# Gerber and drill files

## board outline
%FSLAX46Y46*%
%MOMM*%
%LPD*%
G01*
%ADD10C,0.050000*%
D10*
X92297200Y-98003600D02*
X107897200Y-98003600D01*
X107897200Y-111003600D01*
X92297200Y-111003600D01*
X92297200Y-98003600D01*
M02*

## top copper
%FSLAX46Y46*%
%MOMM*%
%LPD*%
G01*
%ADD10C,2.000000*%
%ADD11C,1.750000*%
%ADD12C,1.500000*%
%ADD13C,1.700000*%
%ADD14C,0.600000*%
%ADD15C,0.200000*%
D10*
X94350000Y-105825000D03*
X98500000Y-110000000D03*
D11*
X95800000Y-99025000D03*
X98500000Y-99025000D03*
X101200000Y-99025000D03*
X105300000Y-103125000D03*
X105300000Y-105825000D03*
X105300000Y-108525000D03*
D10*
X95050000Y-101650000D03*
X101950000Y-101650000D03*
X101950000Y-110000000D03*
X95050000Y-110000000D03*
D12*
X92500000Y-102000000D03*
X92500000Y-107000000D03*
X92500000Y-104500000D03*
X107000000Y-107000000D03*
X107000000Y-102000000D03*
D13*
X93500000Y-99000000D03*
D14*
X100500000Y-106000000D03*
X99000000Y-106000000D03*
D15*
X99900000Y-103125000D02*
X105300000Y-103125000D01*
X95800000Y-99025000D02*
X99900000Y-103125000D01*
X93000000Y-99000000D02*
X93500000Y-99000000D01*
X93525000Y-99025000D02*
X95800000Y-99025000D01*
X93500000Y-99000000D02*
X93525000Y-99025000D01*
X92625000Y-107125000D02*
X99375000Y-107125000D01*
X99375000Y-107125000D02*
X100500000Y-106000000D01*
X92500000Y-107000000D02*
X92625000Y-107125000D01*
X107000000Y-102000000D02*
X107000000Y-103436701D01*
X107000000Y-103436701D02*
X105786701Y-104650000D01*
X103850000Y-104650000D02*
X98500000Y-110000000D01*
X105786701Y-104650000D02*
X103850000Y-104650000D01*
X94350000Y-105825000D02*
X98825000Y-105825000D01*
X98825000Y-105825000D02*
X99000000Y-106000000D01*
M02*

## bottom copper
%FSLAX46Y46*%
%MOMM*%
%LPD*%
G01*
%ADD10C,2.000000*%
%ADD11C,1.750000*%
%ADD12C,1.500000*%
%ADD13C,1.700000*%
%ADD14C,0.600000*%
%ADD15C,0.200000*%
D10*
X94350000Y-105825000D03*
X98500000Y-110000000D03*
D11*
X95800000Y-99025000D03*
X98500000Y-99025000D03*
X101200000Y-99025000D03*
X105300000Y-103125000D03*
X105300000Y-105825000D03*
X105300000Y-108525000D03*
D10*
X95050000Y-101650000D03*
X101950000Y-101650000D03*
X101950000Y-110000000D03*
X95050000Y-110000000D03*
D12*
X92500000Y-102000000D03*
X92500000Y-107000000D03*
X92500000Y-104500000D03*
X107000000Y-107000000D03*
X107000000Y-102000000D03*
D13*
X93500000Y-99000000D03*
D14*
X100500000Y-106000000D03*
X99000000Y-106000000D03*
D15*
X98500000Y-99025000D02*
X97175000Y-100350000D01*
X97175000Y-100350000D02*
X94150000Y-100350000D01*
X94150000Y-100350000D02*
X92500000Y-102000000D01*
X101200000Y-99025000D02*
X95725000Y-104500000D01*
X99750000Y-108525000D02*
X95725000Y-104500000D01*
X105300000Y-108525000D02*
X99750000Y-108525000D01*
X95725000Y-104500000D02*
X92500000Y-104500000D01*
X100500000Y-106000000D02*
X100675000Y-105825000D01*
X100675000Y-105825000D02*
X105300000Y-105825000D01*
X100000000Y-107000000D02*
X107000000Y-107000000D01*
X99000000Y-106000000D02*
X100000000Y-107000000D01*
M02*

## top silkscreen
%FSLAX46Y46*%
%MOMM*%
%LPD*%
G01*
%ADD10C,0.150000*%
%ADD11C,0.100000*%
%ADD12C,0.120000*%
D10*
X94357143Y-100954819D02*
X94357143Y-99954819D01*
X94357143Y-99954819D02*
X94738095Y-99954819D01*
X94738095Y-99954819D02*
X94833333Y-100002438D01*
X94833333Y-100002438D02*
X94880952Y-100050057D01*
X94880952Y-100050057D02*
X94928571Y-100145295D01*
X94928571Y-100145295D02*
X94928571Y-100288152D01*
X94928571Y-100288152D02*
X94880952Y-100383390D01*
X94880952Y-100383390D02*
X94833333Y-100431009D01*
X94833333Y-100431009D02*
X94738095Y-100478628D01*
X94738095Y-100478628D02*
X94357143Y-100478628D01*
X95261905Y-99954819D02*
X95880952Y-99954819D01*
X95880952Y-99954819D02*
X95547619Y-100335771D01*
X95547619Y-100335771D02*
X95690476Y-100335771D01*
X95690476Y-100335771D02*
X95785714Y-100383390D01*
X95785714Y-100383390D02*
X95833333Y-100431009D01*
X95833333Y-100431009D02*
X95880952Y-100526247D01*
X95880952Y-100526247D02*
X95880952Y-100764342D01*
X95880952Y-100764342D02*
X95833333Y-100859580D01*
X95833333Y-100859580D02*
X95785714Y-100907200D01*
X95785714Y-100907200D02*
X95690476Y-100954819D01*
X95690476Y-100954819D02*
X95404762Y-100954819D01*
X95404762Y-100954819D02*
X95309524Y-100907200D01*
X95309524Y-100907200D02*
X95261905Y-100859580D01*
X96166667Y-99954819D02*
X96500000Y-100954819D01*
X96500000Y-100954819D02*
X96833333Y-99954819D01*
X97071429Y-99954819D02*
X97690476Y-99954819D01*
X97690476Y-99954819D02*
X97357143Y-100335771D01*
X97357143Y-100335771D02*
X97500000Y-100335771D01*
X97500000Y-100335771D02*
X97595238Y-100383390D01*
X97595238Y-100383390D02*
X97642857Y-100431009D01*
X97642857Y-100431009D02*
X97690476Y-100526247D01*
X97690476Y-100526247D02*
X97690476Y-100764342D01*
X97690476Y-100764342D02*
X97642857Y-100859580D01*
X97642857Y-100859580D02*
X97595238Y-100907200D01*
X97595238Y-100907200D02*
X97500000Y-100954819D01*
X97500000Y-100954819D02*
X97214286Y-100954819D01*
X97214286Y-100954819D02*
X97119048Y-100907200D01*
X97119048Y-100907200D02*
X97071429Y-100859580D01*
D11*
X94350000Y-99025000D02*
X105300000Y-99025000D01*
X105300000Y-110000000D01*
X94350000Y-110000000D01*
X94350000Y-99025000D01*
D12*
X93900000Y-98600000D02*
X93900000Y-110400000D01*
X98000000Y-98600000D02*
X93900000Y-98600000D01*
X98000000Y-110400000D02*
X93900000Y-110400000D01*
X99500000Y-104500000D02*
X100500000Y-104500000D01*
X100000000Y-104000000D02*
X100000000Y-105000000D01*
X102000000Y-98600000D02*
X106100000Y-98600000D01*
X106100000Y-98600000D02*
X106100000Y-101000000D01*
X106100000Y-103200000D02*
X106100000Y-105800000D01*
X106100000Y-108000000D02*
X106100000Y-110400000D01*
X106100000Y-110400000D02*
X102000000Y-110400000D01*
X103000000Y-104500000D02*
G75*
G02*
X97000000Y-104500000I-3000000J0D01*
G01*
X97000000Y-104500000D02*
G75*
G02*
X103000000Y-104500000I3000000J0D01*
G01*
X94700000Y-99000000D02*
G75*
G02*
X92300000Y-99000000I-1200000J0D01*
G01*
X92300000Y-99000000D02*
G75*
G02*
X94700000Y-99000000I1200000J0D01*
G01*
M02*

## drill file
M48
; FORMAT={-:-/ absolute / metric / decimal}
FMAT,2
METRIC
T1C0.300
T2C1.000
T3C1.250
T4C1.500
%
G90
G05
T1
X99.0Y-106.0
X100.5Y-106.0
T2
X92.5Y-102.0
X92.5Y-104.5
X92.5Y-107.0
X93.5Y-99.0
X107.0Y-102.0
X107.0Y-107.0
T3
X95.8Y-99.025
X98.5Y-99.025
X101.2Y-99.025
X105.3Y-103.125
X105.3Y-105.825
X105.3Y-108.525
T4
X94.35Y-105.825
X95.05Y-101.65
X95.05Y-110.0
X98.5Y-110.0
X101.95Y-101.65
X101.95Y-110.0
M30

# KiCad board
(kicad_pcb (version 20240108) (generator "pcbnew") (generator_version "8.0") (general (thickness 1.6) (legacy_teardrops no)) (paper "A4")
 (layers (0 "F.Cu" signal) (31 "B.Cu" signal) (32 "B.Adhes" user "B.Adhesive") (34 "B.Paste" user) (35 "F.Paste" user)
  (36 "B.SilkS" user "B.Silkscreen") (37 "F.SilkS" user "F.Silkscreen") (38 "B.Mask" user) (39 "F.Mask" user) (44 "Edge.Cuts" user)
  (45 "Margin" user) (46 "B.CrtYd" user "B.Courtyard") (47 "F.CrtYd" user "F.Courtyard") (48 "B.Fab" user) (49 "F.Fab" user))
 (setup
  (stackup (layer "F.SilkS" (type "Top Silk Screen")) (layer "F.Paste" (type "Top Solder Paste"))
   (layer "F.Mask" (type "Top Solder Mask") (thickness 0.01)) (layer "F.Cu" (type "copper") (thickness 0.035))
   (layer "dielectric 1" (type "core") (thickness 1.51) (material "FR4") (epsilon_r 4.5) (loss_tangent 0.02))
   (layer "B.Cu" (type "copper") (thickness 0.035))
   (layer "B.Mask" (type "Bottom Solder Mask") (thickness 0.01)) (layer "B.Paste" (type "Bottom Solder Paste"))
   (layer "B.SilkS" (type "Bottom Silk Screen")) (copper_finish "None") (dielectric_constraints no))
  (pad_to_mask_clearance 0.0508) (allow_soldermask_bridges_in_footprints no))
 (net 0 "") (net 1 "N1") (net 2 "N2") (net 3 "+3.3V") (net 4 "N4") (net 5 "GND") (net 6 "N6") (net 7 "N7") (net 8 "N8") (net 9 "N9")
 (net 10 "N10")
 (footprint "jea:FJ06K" (layer "F.Cu") (at 98.5 105.825)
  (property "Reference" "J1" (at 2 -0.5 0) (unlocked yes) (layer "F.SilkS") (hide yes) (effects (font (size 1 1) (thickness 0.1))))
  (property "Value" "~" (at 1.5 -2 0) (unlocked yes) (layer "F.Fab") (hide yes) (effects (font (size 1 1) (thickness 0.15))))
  (fp_rect (start -4.15 -6.8) (end 6.8 4.175) (stroke (width 0.1) (type default)) (fill none) (layer "F.SilkS"))
  (pad "1" thru_hole circle (at -4.15 0) (size 2 2) (drill 1.5) (layers "*.Cu" "*.Mask") (remove_unused_layers no) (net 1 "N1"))
  (pad "2" thru_hole circle (at 0 4.175) (size 2 2) (drill 1.5) (layers "*.Cu" "*.Mask") (remove_unused_layers no) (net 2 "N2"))
  (pad "3" thru_hole circle (at -2.7 -6.8) (size 1.75 1.75) (drill 1.25) (layers "*.Cu" "*.Mask") (remove_unused_layers no) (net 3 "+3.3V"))
  (pad "4" thru_hole circle (at 0 -6.8) (size 1.75 1.75) (drill 1.25) (layers "*.Cu" "*.Mask") (remove_unused_layers no) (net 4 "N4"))
  (pad "5" thru_hole circle (at 2.7 -6.8) (size 1.75 1.75) (drill 1.25) (layers "*.Cu" "*.Mask") (remove_unused_layers no) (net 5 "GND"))
  (pad "6" thru_hole circle (at 6.8 -2.7) (size 1.75 1.75) (drill 1.25) (layers "*.Cu" "*.Mask") (remove_unused_layers no) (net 3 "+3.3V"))
  (pad "7" thru_hole circle (at 6.8 0) (size 1.75 1.75) (drill 1.25) (layers "*.Cu" "*.Mask") (remove_unused_layers no) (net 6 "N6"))
  (pad "8" thru_hole circle (at 6.8 2.7) (size 1.75 1.75) (drill 1.25) (layers "*.Cu" "*.Mask") (remove_unused_layers no) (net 5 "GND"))
  (pad "9" thru_hole circle (at -3.45 -4.175) (size 2 2) (drill 1.5) (layers "*.Cu" "*.Mask") (remove_unused_layers no) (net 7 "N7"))
  (pad "10" thru_hole circle (at 3.45 -4.175) (size 2 2) (drill 1.5) (layers "*.Cu" "*.Mask") (remove_unused_layers no) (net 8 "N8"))
  (pad "11" thru_hole circle (at 3.45 4.175) (size 2 2) (drill 1.5) (layers "*.Cu" "*.Mask") (remove_unused_layers no) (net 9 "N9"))
  (pad "12" thru_hole circle (at -3.45 4.175) (size 2 2) (drill 1.5) (layers "*.Cu" "*.Mask") (remove_unused_layers no) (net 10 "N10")))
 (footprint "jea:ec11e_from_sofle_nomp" (layer "F.Cu") (at 100 104.5)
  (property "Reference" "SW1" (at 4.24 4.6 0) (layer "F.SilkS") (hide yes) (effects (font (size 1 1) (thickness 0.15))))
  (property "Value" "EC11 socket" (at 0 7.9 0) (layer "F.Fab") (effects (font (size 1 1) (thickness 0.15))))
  (fp_line (start -6.1 -5.9) (end -6.1 5.9) (stroke (width 0.12) (type solid)) (layer "F.SilkS"))
  (fp_line (start -2 -5.9) (end -6.1 -5.9) (stroke (width 0.12) (type solid)) (layer "F.SilkS"))
  (fp_line (start -2 5.9) (end -6.1 5.9) (stroke (width 0.12) (type solid)) (layer "F.SilkS"))
  (fp_line (start -0.5 0) (end 0.5 0) (stroke (width 0.12) (type solid)) (layer "F.SilkS"))
  (fp_line (start 0 -0.5) (end 0 0.5) (stroke (width 0.12) (type solid)) (layer "F.SilkS"))
  (fp_line (start 2 -5.9) (end 6.1 -5.9) (stroke (width 0.12) (type solid)) (layer "F.SilkS"))
  (fp_line (start 6.1 -5.9) (end 6.1 -3.5) (stroke (width 0.12) (type solid)) (layer "F.SilkS"))
  (fp_line (start 6.1 -1.3) (end 6.1 1.3) (stroke (width 0.12) (type solid)) (layer "F.SilkS"))
  (fp_line (start 6.1 3.5) (end 6.1 5.9) (stroke (width 0.12) (type solid)) (layer "F.SilkS"))
  (fp_line (start 6.1 5.9) (end 2 5.9) (stroke (width 0.12) (type solid)) (layer "F.SilkS"))
  (fp_circle (center 0 0) (end 3 0) (stroke (width 0.12) (type solid)) (fill none) (layer "F.SilkS"))
  (pad "A" thru_hole circle (at -7.5 -2.5) (size 1.5 1.5) (drill 1) (layers "*.Cu" "*.Mask") (remove_unused_layers no) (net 4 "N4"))
  (pad "B" thru_hole circle (at -7.5 2.5) (size 1.5 1.5) (drill 1) (layers "*.Cu" "*.Mask") (remove_unused_layers no) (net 6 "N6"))
  (pad "C" thru_hole circle (at -7.5 0) (size 1.5 1.5) (drill 1) (layers "*.Cu" "*.Mask") (remove_unused_layers no) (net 5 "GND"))
  (pad "S1" thru_hole circle (at 7 2.5) (size 1.5 1.5) (drill 1) (layers "*.Cu" "*.Mask") (remove_unused_layers no) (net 1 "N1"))
  (pad "S2" thru_hole circle (at 7 -2.5) (size 1.5 1.5) (drill 1) (layers "*.Cu" "*.Mask") (remove_unused_layers no) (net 2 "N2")))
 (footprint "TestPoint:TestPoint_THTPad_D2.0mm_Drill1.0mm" (layer "F.Cu") (at 93.5 99)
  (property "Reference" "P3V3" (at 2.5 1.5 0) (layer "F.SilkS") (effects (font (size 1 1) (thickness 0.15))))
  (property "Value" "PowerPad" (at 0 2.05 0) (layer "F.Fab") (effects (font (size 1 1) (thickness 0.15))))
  (fp_circle (center 0 0) (end 0 1.2) (stroke (width 0.12) (type solid)) (fill none) (layer "F.SilkS"))
  (pad "1" thru_hole circle (at 0 0) (size 1.7 1.7) (drill 1) (layers "*.Cu" "*.Mask") (remove_unused_layers no) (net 3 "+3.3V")))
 (gr_rect (start 92.2972 98.0036) (end 107.8972 111.0036) (stroke (width 0.05) (type default)) (fill none) (layer "Edge.Cuts"))
 (segment (start 98.5 99.025) (end 97.175 100.35) (width 0.2) (layer "B.Cu") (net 4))
 (segment (start 97.175 100.35) (end 94.15 100.35) (width 0.2) (layer "B.Cu") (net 4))
 (segment (start 94.15 100.35) (end 92.5 102) (width 0.2) (layer "B.Cu") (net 4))
 (segment (start 101.2 99.025) (end 95.725 104.5) (width 0.2) (layer "B.Cu") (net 5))
 (segment (start 99.75 108.525) (end 95.725 104.5) (width 0.2) (layer "B.Cu") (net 5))
 (segment (start 105.3 108.525) (end 99.75 108.525) (width 0.2) (layer "B.Cu") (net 5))
 (segment (start 95.725 104.5) (end 92.5 104.5) (width 0.2) (layer "B.Cu") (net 5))
 (segment (start 99.9 103.125) (end 105.3 103.125) (width 0.2) (layer "F.Cu") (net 3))
 (segment (start 95.8 99.025) (end 99.9 103.125) (width 0.2) (layer "F.Cu") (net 3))
 (segment (start 93 99) (end 93.5 99) (width 0.2) (layer "F.Cu") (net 3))
 (segment (start 93.525 99.025) (end 95.8 99.025) (width 0.2) (layer "F.Cu") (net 3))
 (segment (start 93.5 99) (end 93.525 99.025) (width 0.2) (layer "F.Cu") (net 3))
 (segment (start 92.625 107.125) (end 99.375 107.125) (width 0.2) (layer "F.Cu") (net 6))
 (segment (start 99.375 107.125) (end 100.5 106) (width 0.2) (layer "F.Cu") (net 6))
 (segment (start 92.5 107) (end 92.625 107.125) (width 0.2) (layer "F.Cu") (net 6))
 (via (at 100.5 106) (size 0.6) (drill 0.3) (layers "F.Cu" "B.Cu") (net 6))
 (segment (start 100.5 106) (end 100.675 105.825) (width 0.2) (layer "B.Cu") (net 6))
 (segment (start 100.675 105.825) (end 105.3 105.825) (width 0.2) (layer "B.Cu") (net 6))
 (segment (start 107 102) (end 107 103.436701) (width 0.2) (layer "F.Cu") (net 2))
 (segment (start 107 103.436701) (end 105.786701 104.65) (width 0.2) (layer "F.Cu") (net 2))
 (segment (start 103.85 104.65) (end 98.5 110) (width 0.2) (layer "F.Cu") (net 2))
 (segment (start 105.786701 104.65) (end 103.85 104.65) (width 0.2) (layer "F.Cu") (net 2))
 (segment (start 94.35 105.825) (end 98.825 105.825) (width 0.2) (layer "F.Cu") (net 1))
 (segment (start 98.825 105.825) (end 99 106) (width 0.2) (layer "F.Cu") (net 1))
 (via (at 99 106) (size 0.6) (drill 0.3) (layers "F.Cu" "B.Cu") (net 1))
 (segment (start 100 107) (end 107 107) (width 0.2) (layer "B.Cu") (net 1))
 (segment (start 99 106) (end 100 107) (width 0.2) (layer "B.Cu") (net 1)))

